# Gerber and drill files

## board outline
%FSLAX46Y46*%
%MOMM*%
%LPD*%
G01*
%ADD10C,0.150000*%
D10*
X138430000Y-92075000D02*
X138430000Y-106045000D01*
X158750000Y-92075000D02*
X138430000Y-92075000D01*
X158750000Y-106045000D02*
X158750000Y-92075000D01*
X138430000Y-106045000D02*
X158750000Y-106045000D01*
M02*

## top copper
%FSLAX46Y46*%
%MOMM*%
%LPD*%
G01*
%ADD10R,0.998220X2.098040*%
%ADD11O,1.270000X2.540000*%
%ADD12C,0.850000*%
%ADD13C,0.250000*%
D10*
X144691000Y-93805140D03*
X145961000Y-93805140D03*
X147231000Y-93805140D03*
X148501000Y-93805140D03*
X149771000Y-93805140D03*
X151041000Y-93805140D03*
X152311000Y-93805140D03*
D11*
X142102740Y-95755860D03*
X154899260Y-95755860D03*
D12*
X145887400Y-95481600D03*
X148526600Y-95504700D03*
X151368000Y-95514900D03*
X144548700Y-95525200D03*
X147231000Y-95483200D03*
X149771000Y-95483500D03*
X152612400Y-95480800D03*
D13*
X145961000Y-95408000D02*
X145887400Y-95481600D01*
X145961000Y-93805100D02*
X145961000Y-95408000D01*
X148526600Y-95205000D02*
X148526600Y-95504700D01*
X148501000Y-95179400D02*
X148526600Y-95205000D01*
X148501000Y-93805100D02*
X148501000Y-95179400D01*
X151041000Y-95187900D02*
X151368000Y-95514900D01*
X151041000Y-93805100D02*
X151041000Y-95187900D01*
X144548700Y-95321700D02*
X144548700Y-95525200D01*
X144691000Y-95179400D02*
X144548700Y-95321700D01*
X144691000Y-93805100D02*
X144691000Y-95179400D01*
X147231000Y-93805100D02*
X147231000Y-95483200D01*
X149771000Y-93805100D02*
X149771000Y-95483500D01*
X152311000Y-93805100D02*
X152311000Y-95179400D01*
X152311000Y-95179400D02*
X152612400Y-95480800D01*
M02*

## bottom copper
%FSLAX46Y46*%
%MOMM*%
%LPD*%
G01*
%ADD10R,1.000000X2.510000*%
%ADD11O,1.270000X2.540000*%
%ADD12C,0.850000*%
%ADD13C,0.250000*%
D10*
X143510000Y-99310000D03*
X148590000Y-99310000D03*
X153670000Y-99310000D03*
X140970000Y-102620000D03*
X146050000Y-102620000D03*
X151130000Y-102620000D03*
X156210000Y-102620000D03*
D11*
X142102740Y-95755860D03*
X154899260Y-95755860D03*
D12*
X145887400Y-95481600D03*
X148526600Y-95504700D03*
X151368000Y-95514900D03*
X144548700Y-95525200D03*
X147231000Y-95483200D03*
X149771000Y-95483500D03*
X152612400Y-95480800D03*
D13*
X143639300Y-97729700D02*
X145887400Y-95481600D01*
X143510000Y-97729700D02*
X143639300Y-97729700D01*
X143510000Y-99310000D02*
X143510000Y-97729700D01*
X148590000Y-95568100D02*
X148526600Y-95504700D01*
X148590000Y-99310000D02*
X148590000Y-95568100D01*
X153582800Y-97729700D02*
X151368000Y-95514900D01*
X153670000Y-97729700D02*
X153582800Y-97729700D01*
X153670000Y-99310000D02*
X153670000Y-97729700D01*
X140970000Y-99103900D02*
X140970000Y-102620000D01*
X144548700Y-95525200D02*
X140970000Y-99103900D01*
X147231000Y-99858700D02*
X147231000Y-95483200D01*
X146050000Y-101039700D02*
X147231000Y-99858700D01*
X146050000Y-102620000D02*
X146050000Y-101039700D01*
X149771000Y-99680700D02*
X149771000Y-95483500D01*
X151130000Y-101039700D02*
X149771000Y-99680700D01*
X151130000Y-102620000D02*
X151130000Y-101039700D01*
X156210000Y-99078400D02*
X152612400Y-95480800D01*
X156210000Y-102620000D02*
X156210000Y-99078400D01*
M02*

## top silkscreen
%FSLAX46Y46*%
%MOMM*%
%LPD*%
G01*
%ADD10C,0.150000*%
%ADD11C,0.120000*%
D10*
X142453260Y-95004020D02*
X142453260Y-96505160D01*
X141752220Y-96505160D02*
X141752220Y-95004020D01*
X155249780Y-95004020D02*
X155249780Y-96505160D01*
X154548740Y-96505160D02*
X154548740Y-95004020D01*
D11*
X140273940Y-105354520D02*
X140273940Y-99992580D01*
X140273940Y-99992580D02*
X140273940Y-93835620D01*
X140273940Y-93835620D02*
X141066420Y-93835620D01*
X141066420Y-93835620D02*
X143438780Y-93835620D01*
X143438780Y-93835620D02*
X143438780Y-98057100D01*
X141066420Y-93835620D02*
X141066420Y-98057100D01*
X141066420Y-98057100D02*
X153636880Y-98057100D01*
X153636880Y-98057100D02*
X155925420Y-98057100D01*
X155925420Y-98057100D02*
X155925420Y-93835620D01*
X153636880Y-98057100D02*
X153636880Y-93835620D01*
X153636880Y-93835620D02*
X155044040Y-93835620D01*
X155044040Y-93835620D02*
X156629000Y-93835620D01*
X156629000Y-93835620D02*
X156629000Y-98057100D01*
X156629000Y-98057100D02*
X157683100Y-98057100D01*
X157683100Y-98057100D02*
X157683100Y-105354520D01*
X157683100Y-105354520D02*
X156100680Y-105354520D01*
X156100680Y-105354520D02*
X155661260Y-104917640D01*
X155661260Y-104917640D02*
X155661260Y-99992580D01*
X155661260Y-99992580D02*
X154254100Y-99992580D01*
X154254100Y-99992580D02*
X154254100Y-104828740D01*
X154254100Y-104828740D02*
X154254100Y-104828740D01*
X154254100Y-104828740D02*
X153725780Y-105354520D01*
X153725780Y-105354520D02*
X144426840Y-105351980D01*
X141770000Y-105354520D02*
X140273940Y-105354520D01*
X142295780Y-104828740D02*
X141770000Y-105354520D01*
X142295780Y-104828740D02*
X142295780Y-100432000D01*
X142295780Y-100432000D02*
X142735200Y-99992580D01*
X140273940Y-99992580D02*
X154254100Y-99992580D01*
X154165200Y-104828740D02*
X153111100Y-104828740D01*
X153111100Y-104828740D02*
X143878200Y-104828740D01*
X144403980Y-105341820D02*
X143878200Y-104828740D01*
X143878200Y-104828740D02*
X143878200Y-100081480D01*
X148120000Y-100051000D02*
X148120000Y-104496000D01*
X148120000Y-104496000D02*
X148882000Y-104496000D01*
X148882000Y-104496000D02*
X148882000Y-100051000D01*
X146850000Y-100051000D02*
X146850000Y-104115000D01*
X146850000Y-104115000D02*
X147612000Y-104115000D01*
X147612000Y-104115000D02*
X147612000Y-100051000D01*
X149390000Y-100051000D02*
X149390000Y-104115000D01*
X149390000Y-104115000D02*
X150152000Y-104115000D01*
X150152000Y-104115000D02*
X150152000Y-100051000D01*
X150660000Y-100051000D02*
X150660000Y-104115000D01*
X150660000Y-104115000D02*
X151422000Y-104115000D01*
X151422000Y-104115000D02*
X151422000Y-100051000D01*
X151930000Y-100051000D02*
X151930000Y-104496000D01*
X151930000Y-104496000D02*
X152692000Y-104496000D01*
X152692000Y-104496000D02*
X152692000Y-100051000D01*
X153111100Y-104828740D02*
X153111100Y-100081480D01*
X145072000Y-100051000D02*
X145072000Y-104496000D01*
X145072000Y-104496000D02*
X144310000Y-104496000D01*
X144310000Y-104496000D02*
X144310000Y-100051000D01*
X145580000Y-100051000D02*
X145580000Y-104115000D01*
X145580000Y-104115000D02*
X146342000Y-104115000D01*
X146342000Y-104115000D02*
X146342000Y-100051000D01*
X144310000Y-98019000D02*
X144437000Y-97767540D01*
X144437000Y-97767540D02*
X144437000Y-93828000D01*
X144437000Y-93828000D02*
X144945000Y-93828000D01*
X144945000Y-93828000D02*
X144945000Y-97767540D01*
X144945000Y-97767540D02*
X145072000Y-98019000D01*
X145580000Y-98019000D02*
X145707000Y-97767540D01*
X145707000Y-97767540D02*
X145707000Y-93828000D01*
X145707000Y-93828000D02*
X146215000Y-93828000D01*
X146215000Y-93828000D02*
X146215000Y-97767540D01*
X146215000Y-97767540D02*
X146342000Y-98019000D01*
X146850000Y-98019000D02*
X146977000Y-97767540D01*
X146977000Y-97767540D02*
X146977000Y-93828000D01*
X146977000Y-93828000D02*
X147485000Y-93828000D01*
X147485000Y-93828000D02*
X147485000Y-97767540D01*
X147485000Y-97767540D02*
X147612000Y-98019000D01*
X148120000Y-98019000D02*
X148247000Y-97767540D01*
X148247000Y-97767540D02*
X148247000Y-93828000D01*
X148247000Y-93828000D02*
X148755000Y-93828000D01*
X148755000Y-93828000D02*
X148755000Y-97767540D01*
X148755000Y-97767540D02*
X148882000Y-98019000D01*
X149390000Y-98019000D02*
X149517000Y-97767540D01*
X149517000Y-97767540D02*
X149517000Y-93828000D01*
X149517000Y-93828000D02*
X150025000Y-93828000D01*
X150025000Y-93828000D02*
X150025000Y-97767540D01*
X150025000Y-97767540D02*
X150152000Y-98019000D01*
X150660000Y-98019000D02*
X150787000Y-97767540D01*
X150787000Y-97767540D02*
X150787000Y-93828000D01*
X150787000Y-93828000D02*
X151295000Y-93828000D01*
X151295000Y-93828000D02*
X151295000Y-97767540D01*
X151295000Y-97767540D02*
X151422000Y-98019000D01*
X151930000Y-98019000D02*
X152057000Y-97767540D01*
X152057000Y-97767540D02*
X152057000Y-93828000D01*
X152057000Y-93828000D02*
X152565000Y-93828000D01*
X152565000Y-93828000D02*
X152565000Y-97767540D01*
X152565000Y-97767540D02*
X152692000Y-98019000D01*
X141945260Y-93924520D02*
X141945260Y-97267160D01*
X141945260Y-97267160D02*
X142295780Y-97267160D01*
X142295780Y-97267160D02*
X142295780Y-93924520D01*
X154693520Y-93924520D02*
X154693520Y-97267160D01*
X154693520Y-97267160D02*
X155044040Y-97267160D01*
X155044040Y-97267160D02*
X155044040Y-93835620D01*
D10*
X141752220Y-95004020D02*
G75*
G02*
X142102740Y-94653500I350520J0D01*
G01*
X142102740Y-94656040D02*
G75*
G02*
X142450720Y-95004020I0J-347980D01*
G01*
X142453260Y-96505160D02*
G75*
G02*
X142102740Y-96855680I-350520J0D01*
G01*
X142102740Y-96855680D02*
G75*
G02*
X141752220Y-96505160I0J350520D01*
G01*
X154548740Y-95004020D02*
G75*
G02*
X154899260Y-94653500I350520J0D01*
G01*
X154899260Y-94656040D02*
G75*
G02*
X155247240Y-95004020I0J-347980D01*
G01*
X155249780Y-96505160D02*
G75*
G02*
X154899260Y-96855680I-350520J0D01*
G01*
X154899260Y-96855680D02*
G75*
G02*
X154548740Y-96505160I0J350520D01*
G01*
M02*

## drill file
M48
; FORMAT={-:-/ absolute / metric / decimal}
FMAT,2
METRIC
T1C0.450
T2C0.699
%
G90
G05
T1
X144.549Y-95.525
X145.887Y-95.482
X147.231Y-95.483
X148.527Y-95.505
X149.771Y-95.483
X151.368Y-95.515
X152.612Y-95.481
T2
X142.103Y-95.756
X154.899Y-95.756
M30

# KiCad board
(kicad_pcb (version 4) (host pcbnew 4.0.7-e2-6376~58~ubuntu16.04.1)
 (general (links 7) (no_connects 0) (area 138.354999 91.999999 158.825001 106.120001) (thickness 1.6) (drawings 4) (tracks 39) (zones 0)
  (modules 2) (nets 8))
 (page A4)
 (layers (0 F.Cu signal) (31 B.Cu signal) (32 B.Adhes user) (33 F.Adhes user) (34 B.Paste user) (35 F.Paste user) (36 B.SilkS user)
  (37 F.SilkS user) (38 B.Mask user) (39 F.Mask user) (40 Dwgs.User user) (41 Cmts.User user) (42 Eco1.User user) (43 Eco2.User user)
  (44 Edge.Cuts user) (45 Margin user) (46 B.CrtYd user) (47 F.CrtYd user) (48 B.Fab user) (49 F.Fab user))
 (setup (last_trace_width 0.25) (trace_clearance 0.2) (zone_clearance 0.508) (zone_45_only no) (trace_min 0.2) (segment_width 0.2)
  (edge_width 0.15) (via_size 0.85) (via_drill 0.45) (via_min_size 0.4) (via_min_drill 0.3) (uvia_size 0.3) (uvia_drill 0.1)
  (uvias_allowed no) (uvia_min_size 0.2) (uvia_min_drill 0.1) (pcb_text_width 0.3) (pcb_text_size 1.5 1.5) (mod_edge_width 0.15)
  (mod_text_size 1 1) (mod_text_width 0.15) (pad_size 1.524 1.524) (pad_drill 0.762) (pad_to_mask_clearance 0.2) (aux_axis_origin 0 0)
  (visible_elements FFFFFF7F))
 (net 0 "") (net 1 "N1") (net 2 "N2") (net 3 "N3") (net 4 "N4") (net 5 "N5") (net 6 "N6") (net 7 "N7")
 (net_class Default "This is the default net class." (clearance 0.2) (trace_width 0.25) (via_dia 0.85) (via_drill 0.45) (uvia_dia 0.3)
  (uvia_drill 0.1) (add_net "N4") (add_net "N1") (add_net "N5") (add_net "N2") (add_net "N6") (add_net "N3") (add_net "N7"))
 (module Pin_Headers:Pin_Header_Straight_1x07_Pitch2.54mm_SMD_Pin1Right (layer B.Cu) (at 148.59 100.965 270)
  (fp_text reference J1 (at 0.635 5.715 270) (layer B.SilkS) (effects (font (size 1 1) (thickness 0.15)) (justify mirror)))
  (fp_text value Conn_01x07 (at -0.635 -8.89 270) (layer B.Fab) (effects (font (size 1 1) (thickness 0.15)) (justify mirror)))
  (pad 2 smd rect (at -1.655 5.08 270) (size 2.51 1) (layers B.Cu B.Paste B.Mask) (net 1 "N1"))
  (pad 4 smd rect (at -1.655 0 270) (size 2.51 1) (layers B.Cu B.Paste B.Mask) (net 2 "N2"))
  (pad 6 smd rect (at -1.655 -5.08 270) (size 2.51 1) (layers B.Cu B.Paste B.Mask) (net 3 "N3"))
  (pad 1 smd rect (at 1.655 7.62 270) (size 2.51 1) (layers B.Cu B.Paste B.Mask) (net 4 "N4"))
  (pad 3 smd rect (at 1.655 2.54 270) (size 2.51 1) (layers B.Cu B.Paste B.Mask) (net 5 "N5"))
  (pad 5 smd rect (at 1.655 -2.54 270) (size 2.51 1) (layers B.Cu B.Paste B.Mask) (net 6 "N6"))
  (pad 7 smd rect (at 1.655 -7.62 270) (size 2.51 1) (layers B.Cu B.Paste B.Mask) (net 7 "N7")))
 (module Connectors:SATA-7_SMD (layer F.Cu) (at 148.501 105.004)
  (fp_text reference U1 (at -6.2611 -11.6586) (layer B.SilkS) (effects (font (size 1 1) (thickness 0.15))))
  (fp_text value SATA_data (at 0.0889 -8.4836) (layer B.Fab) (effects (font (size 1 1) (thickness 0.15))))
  (fp_line (start -6.04774 -9.99998) (end -6.04774 -8.49884) (layer F.SilkS) (width 0.15))
  (fp_line (start -6.74878 -8.49884) (end -6.74878 -9.99998) (layer F.SilkS) (width 0.15))
  (fp_line (start 6.74878 -9.99998) (end 6.74878 -8.49884) (layer F.SilkS) (width 0.15))
  (fp_line (start 6.04774 -8.49884) (end 6.04774 -9.99998) (layer F.SilkS) (width 0.15))
  (fp_line (start -8.22706 0.35052) (end -8.22706 -5.01142) (layer F.SilkS) (width 0.12))
  (fp_line (start -8.22706 -5.01142) (end -8.22706 -11.16838) (layer F.SilkS) (width 0.12))
  (fp_line (start -8.22706 -11.16838) (end -7.43458 -11.16838) (layer F.SilkS) (width 0.12))
  (fp_line (start -7.43458 -11.16838) (end -5.06222 -11.16838) (layer F.SilkS) (width 0.12))
  (fp_line (start -5.06222 -11.16838) (end -5.06222 -6.9469) (layer F.SilkS) (width 0.12))
  (fp_line (start -7.43458 -11.16838) (end -7.43458 -6.9469) (layer F.SilkS) (width 0.12))
  (fp_line (start -7.43458 -6.9469) (end 5.13588 -6.9469) (layer F.SilkS) (width 0.12))
  (fp_line (start 5.13588 -6.9469) (end 7.42442 -6.9469) (layer F.SilkS) (width 0.12))
  (fp_line (start 7.42442 -6.9469) (end 7.42442 -11.16838) (layer F.SilkS) (width 0.12))
  (fp_line (start 5.13588 -6.9469) (end 5.13588 -11.16838) (layer F.SilkS) (width 0.12))
  (fp_line (start 5.13588 -11.16838) (end 6.54304 -11.16838) (layer F.SilkS) (width 0.12))
  (fp_line (start 6.54304 -11.16838) (end 8.128 -11.16838) (layer F.SilkS) (width 0.12))
  (fp_line (start 8.128 -11.16838) (end 8.128 -6.9469) (layer F.SilkS) (width 0.12))
  (fp_line (start 8.128 -6.9469) (end 9.1821 -6.9469) (layer F.SilkS) (width 0.12))
  (fp_line (start 9.1821 -6.9469) (end 9.1821 0.35052) (layer F.SilkS) (width 0.12))
  (fp_line (start 9.1821 0.35052) (end 7.59968 0.35052) (layer F.SilkS) (width 0.12))
  (fp_line (start 7.59968 0.35052) (end 7.16026 -0.08636) (layer F.SilkS) (width 0.12))
  (fp_line (start 7.16026 -0.08636) (end 7.16026 -5.01142) (layer F.SilkS) (width 0.12))
  (fp_line (start 7.16026 -5.01142) (end 5.7531 -5.01142) (layer F.SilkS) (width 0.12))
  (fp_line (start 5.7531 -5.01142) (end 5.7531 -0.17526) (layer F.SilkS) (width 0.12))
  (fp_line (start 5.7531 -0.17526) (end 5.7531 -0.17526) (layer F.SilkS) (width 0.12))
  (fp_line (start 5.7531 -0.17526) (end 5.22478 0.35052) (layer F.SilkS) (width 0.12))
  (fp_line (start 5.22478 0.35052) (end -4.07416 0.34798) (layer F.SilkS) (width 0.12))
  (fp_line (start -6.731 0.35052) (end -8.22706 0.35052) (layer F.SilkS) (width 0.12))
  (fp_line (start -6.20522 -0.17526) (end -6.731 0.35052) (layer F.SilkS) (width 0.12))
  (fp_line (start -6.20522 -0.17526) (end -6.20522 -4.572) (layer F.SilkS) (width 0.12))
  (fp_line (start -6.20522 -4.572) (end -5.7658 -5.01142) (layer F.SilkS) (width 0.12))
  (fp_line (start -8.22706 -5.01142) (end 5.7531 -5.01142) (layer F.SilkS) (width 0.12))
  (fp_line (start 5.6642 -0.17526) (end 4.6101 -0.17526) (layer F.SilkS) (width 0.12))
  (fp_line (start 4.6101 -0.17526) (end -4.6228 -0.17526) (layer F.SilkS) (width 0.12))
  (fp_line (start -4.09702 0.33782) (end -4.6228 -0.17526) (layer F.SilkS) (width 0.12))
  (fp_line (start -4.6228 -0.17526) (end -4.6228 -4.92252) (layer F.SilkS) (width 0.12))
  (fp_line (start -0.381 -4.953) (end -0.381 -0.508) (layer F.SilkS) (width 0.12))
  (fp_line (start -0.381 -0.508) (end 0.381 -0.508) (layer F.SilkS) (width 0.12))
  (fp_line (start 0.381 -0.508) (end 0.381 -4.953) (layer F.SilkS) (width 0.12))
  (fp_line (start -1.651 -4.953) (end -1.651 -0.889) (layer F.SilkS) (width 0.12))
  (fp_line (start -1.651 -0.889) (end -0.889 -0.889) (layer F.SilkS) (width 0.12))
  (fp_line (start -0.889 -0.889) (end -0.889 -4.953) (layer F.SilkS) (width 0.12))
  (fp_line (start 0.889 -4.953) (end 0.889 -0.889) (layer F.SilkS) (width 0.12))
  (fp_line (start 0.889 -0.889) (end 1.651 -0.889) (layer F.SilkS) (width 0.12))
  (fp_line (start 1.651 -0.889) (end 1.651 -4.953) (layer F.SilkS) (width 0.12))
  (fp_line (start 2.159 -4.953) (end 2.159 -0.889) (layer F.SilkS) (width 0.12))
  (fp_line (start 2.159 -0.889) (end 2.921 -0.889) (layer F.SilkS) (width 0.12))
  (fp_line (start 2.921 -0.889) (end 2.921 -4.953) (layer F.SilkS) (width 0.12))
  (fp_line (start 3.429 -4.953) (end 3.429 -0.508) (layer F.SilkS) (width 0.12))
  (fp_line (start 3.429 -0.508) (end 4.191 -0.508) (layer F.SilkS) (width 0.12))
  (fp_line (start 4.191 -0.508) (end 4.191 -4.953) (layer F.SilkS) (width 0.12))
  (fp_line (start 4.6101 -0.17526) (end 4.6101 -4.92252) (layer F.SilkS) (width 0.12))
  (fp_line (start -3.429 -4.953) (end -3.429 -0.508) (layer F.SilkS) (width 0.12))
  (fp_line (start -3.429 -0.508) (end -4.191 -0.508) (layer F.SilkS) (width 0.12))
  (fp_line (start -4.191 -0.508) (end -4.191 -4.953) (layer F.SilkS) (width 0.12))
  (fp_line (start -2.921 -4.953) (end -2.921 -0.889) (layer F.SilkS) (width 0.12))
  (fp_line (start -2.921 -0.889) (end -2.159 -0.889) (layer F.SilkS) (width 0.12))
  (fp_line (start -2.159 -0.889) (end -2.159 -4.953) (layer F.SilkS) (width 0.12))
  (fp_line (start -4.191 -6.985) (end -4.064 -7.23646) (layer F.SilkS) (width 0.12))
  (fp_line (start -4.064 -7.23646) (end -4.064 -11.176) (layer F.SilkS) (width 0.12))
  (fp_line (start -4.064 -11.176) (end -3.556 -11.176) (layer F.SilkS) (width 0.12))
  (fp_line (start -3.556 -11.176) (end -3.556 -7.23646) (layer F.SilkS) (width 0.12))
  (fp_line (start -3.556 -7.23646) (end -3.429 -6.985) (layer F.SilkS) (width 0.12))
  (fp_line (start -2.921 -6.985) (end -2.794 -7.23646) (layer F.SilkS) (width 0.12))
  (fp_line (start -2.794 -7.23646) (end -2.794 -11.176) (layer F.SilkS) (width 0.12))
  (fp_line (start -2.794 -11.176) (end -2.286 -11.176) (layer F.SilkS) (width 0.12))
  (fp_line (start -2.286 -11.176) (end -2.286 -7.23646) (layer F.SilkS) (width 0.12))
  (fp_line (start -2.286 -7.23646) (end -2.159 -6.985) (layer F.SilkS) (width 0.12))
  (fp_line (start -1.651 -6.985) (end -1.524 -7.23646) (layer F.SilkS) (width 0.12))
  (fp_line (start -1.524 -7.23646) (end -1.524 -11.176) (layer F.SilkS) (width 0.12))
  (fp_line (start -1.524 -11.176) (end -1.016 -11.176) (layer F.SilkS) (width 0.12))
  (fp_line (start -1.016 -11.176) (end -1.016 -7.23646) (layer F.SilkS) (width 0.12))
  (fp_line (start -1.016 -7.23646) (end -0.889 -6.985) (layer F.SilkS) (width 0.12))
  (fp_line (start -0.381 -6.985) (end -0.254 -7.23646) (layer F.SilkS) (width 0.12))
  (fp_line (start -0.254 -7.23646) (end -0.254 -11.176) (layer F.SilkS) (width 0.12))
  (fp_line (start -0.254 -11.176) (end 0.254 -11.176) (layer F.SilkS) (width 0.12))
  (fp_line (start 0.254 -11.176) (end 0.254 -7.23646) (layer F.SilkS) (width 0.12))
  (fp_line (start 0.254 -7.23646) (end 0.381 -6.985) (layer F.SilkS) (width 0.12))
  (fp_line (start 0.889 -6.985) (end 1.016 -7.23646) (layer F.SilkS) (width 0.12))
  (fp_line (start 1.016 -7.23646) (end 1.016 -11.176) (layer F.SilkS) (width 0.12))
  (fp_line (start 1.016 -11.176) (end 1.524 -11.176) (layer F.SilkS) (width 0.12))
  (fp_line (start 1.524 -11.176) (end 1.524 -7.23646) (layer F.SilkS) (width 0.12))
  (fp_line (start 1.524 -7.23646) (end 1.651 -6.985) (layer F.SilkS) (width 0.12))
  (fp_line (start 2.159 -6.985) (end 2.286 -7.23646) (layer F.SilkS) (width 0.12))
  (fp_line (start 2.286 -7.23646) (end 2.286 -11.176) (layer F.SilkS) (width 0.12))
  (fp_line (start 2.286 -11.176) (end 2.794 -11.176) (layer F.SilkS) (width 0.12))
  (fp_line (start 2.794 -11.176) (end 2.794 -7.23646) (layer F.SilkS) (width 0.12))
  (fp_line (start 2.794 -7.23646) (end 2.921 -6.985) (layer F.SilkS) (width 0.12))
  (fp_line (start 3.429 -6.985) (end 3.556 -7.23646) (layer F.SilkS) (width 0.12))
  (fp_line (start 3.556 -7.23646) (end 3.556 -11.176) (layer F.SilkS) (width 0.12))
  (fp_line (start 3.556 -11.176) (end 4.064 -11.176) (layer F.SilkS) (width 0.12))
  (fp_line (start 4.064 -11.176) (end 4.064 -7.23646) (layer F.SilkS) (width 0.12))
  (fp_line (start 4.064 -7.23646) (end 4.191 -6.985) (layer F.SilkS) (width 0.12))
  (fp_line (start -6.55574 -11.07948) (end -6.55574 -7.73684) (layer F.SilkS) (width 0.12))
  (fp_line (start -6.55574 -7.73684) (end -6.20522 -7.73684) (layer F.SilkS) (width 0.12))
  (fp_line (start -6.20522 -7.73684) (end -6.20522 -11.07948) (layer F.SilkS) (width 0.12))
  (fp_line (start 6.19252 -11.07948) (end 6.19252 -7.73684) (layer F.SilkS) (width 0.12))
  (fp_line (start 6.19252 -7.73684) (end 6.54304 -7.73684) (layer F.SilkS) (width 0.12))
  (fp_line (start 6.54304 -7.73684) (end 6.54304 -11.16838) (layer F.SilkS) (width 0.12))
  (fp_arc (start -6.39826 -9.99998) (end -6.74878 -9.99998) (angle 90) (layer F.SilkS) (width 0.15))
  (fp_arc (start -6.39826 -9.99998) (end -6.39826 -10.34796) (angle 90) (layer F.SilkS) (width 0.15))
  (fp_arc (start -6.39826 -8.49884) (end -6.04774 -8.49884) (angle 90) (layer F.SilkS) (width 0.15))
  (fp_arc (start -6.39826 -8.49884) (end -6.39826 -8.14832) (angle 90) (layer F.SilkS) (width 0.15))
  (fp_arc (start 6.39826 -9.99998) (end 6.04774 -9.99998) (angle 90) (layer F.SilkS) (width 0.15))
  (fp_arc (start 6.39826 -9.99998) (end 6.39826 -10.34796) (angle 90) (layer F.SilkS) (width 0.15))
  (fp_arc (start 6.39826 -8.49884) (end 6.74878 -8.49884) (angle 90) (layer F.SilkS) (width 0.15))
  (fp_arc (start 6.39826 -8.49884) (end 6.39826 -8.14832) (angle 90) (layer F.SilkS) (width 0.15))
  (pad 1 smd rect (at -3.81 -11.19886) (size 0.99822 2.09804) (layers F.Cu F.Paste F.Mask) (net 4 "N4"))
  (pad 2 smd rect (at -2.54 -11.19886) (size 0.99822 2.09804) (layers F.Cu F.Paste F.Mask) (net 1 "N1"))
  (pad 3 smd rect (at -1.27 -11.19886) (size 0.99822 2.09804) (layers F.Cu F.Paste F.Mask) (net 5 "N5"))
  (pad 4 smd rect (at 0 -11.19886) (size 0.99822 2.09804) (layers F.Cu F.Paste F.Mask) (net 2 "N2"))
  (pad 5 smd rect (at 1.27 -11.19886) (size 0.99822 2.09804) (layers F.Cu F.Paste F.Mask) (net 6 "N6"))
  (pad 6 smd rect (at 2.54 -11.19886) (size 0.99822 2.09804) (layers F.Cu F.Paste F.Mask) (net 3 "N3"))
  (pad 7 smd rect (at 3.81 -11.19886) (size 0.99822 2.09804) (layers F.Cu F.Paste F.Mask) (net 7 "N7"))
  (pad M1 thru_hole oval (at -6.39826 -9.24814) (size 1.27 2.54) (drill 0.6985) (layers *.Cu F.Paste F.Mask))
  (pad M2 thru_hole oval (at 6.39826 -9.24814) (size 1.27 2.54) (drill 0.6985) (layers *.Cu F.Paste F.Mask)))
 (gr_line (start 138.43 92.075) (end 138.43 106.045) (layer Edge.Cuts) (width 0.15))
 (gr_line (start 158.75 92.075) (end 138.43 92.075) (layer Edge.Cuts) (width 0.15))
 (gr_line (start 158.75 106.045) (end 158.75 92.075) (layer Edge.Cuts) (width 0.15))
 (gr_line (start 138.43 106.045) (end 158.75 106.045) (layer Edge.Cuts) (width 0.15))
 (via (at 145.8874 95.4816) (size 0.85) (layers F.Cu B.Cu) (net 1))
 (segment (start 143.6393 97.7297) (end 145.8874 95.4816) (width 0.25) (layer B.Cu) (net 1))
 (segment (start 143.51 97.7297) (end 143.6393 97.7297) (width 0.25) (layer B.Cu) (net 1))
 (segment (start 145.961 95.408) (end 145.8874 95.4816) (width 0.25) (layer F.Cu) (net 1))
 (segment (start 145.961 93.8051) (end 145.961 95.408) (width 0.25) (layer F.Cu) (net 1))
 (segment (start 143.51 99.31) (end 143.51 97.7297) (width 0.25) (layer B.Cu) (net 1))
 (via (at 148.5266 95.5047) (size 0.85) (layers F.Cu B.Cu) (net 2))
 (segment (start 148.59 95.5681) (end 148.5266 95.5047) (width 0.25) (layer B.Cu) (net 2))
 (segment (start 148.59 99.31) (end 148.59 95.5681) (width 0.25) (layer B.Cu) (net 2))
 (segment (start 148.5266 95.205) (end 148.5266 95.5047) (width 0.25) (layer F.Cu) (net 2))
 (segment (start 148.501 95.1794) (end 148.5266 95.205) (width 0.25) (layer F.Cu) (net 2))
 (segment (start 148.501 93.8051) (end 148.501 95.1794) (width 0.25) (layer F.Cu) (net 2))
 (via (at 151.368 95.5149) (size 0.85) (layers F.Cu B.Cu) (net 3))
 (segment (start 153.5828 97.7297) (end 151.368 95.5149) (width 0.25) (layer B.Cu) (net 3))
 (segment (start 153.67 97.7297) (end 153.5828 97.7297) (width 0.25) (layer B.Cu) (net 3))
 (segment (start 151.041 95.1879) (end 151.368 95.5149) (width 0.25) (layer F.Cu) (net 3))
 (segment (start 151.041 93.8051) (end 151.041 95.1879) (width 0.25) (layer F.Cu) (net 3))
 (segment (start 153.67 99.31) (end 153.67 97.7297) (width 0.25) (layer B.Cu) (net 3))
 (via (at 144.5487 95.5252) (size 0.85) (layers F.Cu B.Cu) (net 4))
 (segment (start 144.5487 95.3217) (end 144.5487 95.5252) (width 0.25) (layer F.Cu) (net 4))
 (segment (start 144.691 95.1794) (end 144.5487 95.3217) (width 0.25) (layer F.Cu) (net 4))
 (segment (start 140.97 99.1039) (end 140.97 102.62) (width 0.25) (layer B.Cu) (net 4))
 (segment (start 144.5487 95.5252) (end 140.97 99.1039) (width 0.25) (layer B.Cu) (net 4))
 (segment (start 144.691 93.8051) (end 144.691 95.1794) (width 0.25) (layer F.Cu) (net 4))
 (via (at 147.231 95.4832) (size 0.85) (layers F.Cu B.Cu) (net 5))
 (segment (start 147.231 99.8587) (end 147.231 95.4832) (width 0.25) (layer B.Cu) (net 5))
 (segment (start 146.05 101.0397) (end 147.231 99.8587) (width 0.25) (layer B.Cu) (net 5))
 (segment (start 147.231 93.8051) (end 147.231 95.4832) (width 0.25) (layer F.Cu) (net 5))
 (segment (start 146.05 102.62) (end 146.05 101.0397) (width 0.25) (layer B.Cu) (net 5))
 (via (at 149.771 95.4835) (size 0.85) (layers F.Cu B.Cu) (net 6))
 (segment (start 149.771 99.6807) (end 149.771 95.4835) (width 0.25) (layer B.Cu) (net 6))
 (segment (start 151.13 101.0397) (end 149.771 99.6807) (width 0.25) (layer B.Cu) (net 6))
 (segment (start 149.771 93.8051) (end 149.771 95.4835) (width 0.25) (layer F.Cu) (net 6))
 (segment (start 151.13 102.62) (end 151.13 101.0397) (width 0.25) (layer B.Cu) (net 6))
 (via (at 152.6124 95.4808) (size 0.85) (layers F.Cu B.Cu) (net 7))
 (segment (start 152.311 93.8051) (end 152.311 95.1794) (width 0.25) (layer F.Cu) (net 7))
 (segment (start 156.21 99.0784) (end 152.6124 95.4808) (width 0.25) (layer B.Cu) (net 7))
 (segment (start 156.21 102.62) (end 156.21 99.0784) (width 0.25) (layer B.Cu) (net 7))
 (segment (start 152.311 95.1794) (end 152.6124 95.4808) (width 0.25) (layer F.Cu) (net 7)))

